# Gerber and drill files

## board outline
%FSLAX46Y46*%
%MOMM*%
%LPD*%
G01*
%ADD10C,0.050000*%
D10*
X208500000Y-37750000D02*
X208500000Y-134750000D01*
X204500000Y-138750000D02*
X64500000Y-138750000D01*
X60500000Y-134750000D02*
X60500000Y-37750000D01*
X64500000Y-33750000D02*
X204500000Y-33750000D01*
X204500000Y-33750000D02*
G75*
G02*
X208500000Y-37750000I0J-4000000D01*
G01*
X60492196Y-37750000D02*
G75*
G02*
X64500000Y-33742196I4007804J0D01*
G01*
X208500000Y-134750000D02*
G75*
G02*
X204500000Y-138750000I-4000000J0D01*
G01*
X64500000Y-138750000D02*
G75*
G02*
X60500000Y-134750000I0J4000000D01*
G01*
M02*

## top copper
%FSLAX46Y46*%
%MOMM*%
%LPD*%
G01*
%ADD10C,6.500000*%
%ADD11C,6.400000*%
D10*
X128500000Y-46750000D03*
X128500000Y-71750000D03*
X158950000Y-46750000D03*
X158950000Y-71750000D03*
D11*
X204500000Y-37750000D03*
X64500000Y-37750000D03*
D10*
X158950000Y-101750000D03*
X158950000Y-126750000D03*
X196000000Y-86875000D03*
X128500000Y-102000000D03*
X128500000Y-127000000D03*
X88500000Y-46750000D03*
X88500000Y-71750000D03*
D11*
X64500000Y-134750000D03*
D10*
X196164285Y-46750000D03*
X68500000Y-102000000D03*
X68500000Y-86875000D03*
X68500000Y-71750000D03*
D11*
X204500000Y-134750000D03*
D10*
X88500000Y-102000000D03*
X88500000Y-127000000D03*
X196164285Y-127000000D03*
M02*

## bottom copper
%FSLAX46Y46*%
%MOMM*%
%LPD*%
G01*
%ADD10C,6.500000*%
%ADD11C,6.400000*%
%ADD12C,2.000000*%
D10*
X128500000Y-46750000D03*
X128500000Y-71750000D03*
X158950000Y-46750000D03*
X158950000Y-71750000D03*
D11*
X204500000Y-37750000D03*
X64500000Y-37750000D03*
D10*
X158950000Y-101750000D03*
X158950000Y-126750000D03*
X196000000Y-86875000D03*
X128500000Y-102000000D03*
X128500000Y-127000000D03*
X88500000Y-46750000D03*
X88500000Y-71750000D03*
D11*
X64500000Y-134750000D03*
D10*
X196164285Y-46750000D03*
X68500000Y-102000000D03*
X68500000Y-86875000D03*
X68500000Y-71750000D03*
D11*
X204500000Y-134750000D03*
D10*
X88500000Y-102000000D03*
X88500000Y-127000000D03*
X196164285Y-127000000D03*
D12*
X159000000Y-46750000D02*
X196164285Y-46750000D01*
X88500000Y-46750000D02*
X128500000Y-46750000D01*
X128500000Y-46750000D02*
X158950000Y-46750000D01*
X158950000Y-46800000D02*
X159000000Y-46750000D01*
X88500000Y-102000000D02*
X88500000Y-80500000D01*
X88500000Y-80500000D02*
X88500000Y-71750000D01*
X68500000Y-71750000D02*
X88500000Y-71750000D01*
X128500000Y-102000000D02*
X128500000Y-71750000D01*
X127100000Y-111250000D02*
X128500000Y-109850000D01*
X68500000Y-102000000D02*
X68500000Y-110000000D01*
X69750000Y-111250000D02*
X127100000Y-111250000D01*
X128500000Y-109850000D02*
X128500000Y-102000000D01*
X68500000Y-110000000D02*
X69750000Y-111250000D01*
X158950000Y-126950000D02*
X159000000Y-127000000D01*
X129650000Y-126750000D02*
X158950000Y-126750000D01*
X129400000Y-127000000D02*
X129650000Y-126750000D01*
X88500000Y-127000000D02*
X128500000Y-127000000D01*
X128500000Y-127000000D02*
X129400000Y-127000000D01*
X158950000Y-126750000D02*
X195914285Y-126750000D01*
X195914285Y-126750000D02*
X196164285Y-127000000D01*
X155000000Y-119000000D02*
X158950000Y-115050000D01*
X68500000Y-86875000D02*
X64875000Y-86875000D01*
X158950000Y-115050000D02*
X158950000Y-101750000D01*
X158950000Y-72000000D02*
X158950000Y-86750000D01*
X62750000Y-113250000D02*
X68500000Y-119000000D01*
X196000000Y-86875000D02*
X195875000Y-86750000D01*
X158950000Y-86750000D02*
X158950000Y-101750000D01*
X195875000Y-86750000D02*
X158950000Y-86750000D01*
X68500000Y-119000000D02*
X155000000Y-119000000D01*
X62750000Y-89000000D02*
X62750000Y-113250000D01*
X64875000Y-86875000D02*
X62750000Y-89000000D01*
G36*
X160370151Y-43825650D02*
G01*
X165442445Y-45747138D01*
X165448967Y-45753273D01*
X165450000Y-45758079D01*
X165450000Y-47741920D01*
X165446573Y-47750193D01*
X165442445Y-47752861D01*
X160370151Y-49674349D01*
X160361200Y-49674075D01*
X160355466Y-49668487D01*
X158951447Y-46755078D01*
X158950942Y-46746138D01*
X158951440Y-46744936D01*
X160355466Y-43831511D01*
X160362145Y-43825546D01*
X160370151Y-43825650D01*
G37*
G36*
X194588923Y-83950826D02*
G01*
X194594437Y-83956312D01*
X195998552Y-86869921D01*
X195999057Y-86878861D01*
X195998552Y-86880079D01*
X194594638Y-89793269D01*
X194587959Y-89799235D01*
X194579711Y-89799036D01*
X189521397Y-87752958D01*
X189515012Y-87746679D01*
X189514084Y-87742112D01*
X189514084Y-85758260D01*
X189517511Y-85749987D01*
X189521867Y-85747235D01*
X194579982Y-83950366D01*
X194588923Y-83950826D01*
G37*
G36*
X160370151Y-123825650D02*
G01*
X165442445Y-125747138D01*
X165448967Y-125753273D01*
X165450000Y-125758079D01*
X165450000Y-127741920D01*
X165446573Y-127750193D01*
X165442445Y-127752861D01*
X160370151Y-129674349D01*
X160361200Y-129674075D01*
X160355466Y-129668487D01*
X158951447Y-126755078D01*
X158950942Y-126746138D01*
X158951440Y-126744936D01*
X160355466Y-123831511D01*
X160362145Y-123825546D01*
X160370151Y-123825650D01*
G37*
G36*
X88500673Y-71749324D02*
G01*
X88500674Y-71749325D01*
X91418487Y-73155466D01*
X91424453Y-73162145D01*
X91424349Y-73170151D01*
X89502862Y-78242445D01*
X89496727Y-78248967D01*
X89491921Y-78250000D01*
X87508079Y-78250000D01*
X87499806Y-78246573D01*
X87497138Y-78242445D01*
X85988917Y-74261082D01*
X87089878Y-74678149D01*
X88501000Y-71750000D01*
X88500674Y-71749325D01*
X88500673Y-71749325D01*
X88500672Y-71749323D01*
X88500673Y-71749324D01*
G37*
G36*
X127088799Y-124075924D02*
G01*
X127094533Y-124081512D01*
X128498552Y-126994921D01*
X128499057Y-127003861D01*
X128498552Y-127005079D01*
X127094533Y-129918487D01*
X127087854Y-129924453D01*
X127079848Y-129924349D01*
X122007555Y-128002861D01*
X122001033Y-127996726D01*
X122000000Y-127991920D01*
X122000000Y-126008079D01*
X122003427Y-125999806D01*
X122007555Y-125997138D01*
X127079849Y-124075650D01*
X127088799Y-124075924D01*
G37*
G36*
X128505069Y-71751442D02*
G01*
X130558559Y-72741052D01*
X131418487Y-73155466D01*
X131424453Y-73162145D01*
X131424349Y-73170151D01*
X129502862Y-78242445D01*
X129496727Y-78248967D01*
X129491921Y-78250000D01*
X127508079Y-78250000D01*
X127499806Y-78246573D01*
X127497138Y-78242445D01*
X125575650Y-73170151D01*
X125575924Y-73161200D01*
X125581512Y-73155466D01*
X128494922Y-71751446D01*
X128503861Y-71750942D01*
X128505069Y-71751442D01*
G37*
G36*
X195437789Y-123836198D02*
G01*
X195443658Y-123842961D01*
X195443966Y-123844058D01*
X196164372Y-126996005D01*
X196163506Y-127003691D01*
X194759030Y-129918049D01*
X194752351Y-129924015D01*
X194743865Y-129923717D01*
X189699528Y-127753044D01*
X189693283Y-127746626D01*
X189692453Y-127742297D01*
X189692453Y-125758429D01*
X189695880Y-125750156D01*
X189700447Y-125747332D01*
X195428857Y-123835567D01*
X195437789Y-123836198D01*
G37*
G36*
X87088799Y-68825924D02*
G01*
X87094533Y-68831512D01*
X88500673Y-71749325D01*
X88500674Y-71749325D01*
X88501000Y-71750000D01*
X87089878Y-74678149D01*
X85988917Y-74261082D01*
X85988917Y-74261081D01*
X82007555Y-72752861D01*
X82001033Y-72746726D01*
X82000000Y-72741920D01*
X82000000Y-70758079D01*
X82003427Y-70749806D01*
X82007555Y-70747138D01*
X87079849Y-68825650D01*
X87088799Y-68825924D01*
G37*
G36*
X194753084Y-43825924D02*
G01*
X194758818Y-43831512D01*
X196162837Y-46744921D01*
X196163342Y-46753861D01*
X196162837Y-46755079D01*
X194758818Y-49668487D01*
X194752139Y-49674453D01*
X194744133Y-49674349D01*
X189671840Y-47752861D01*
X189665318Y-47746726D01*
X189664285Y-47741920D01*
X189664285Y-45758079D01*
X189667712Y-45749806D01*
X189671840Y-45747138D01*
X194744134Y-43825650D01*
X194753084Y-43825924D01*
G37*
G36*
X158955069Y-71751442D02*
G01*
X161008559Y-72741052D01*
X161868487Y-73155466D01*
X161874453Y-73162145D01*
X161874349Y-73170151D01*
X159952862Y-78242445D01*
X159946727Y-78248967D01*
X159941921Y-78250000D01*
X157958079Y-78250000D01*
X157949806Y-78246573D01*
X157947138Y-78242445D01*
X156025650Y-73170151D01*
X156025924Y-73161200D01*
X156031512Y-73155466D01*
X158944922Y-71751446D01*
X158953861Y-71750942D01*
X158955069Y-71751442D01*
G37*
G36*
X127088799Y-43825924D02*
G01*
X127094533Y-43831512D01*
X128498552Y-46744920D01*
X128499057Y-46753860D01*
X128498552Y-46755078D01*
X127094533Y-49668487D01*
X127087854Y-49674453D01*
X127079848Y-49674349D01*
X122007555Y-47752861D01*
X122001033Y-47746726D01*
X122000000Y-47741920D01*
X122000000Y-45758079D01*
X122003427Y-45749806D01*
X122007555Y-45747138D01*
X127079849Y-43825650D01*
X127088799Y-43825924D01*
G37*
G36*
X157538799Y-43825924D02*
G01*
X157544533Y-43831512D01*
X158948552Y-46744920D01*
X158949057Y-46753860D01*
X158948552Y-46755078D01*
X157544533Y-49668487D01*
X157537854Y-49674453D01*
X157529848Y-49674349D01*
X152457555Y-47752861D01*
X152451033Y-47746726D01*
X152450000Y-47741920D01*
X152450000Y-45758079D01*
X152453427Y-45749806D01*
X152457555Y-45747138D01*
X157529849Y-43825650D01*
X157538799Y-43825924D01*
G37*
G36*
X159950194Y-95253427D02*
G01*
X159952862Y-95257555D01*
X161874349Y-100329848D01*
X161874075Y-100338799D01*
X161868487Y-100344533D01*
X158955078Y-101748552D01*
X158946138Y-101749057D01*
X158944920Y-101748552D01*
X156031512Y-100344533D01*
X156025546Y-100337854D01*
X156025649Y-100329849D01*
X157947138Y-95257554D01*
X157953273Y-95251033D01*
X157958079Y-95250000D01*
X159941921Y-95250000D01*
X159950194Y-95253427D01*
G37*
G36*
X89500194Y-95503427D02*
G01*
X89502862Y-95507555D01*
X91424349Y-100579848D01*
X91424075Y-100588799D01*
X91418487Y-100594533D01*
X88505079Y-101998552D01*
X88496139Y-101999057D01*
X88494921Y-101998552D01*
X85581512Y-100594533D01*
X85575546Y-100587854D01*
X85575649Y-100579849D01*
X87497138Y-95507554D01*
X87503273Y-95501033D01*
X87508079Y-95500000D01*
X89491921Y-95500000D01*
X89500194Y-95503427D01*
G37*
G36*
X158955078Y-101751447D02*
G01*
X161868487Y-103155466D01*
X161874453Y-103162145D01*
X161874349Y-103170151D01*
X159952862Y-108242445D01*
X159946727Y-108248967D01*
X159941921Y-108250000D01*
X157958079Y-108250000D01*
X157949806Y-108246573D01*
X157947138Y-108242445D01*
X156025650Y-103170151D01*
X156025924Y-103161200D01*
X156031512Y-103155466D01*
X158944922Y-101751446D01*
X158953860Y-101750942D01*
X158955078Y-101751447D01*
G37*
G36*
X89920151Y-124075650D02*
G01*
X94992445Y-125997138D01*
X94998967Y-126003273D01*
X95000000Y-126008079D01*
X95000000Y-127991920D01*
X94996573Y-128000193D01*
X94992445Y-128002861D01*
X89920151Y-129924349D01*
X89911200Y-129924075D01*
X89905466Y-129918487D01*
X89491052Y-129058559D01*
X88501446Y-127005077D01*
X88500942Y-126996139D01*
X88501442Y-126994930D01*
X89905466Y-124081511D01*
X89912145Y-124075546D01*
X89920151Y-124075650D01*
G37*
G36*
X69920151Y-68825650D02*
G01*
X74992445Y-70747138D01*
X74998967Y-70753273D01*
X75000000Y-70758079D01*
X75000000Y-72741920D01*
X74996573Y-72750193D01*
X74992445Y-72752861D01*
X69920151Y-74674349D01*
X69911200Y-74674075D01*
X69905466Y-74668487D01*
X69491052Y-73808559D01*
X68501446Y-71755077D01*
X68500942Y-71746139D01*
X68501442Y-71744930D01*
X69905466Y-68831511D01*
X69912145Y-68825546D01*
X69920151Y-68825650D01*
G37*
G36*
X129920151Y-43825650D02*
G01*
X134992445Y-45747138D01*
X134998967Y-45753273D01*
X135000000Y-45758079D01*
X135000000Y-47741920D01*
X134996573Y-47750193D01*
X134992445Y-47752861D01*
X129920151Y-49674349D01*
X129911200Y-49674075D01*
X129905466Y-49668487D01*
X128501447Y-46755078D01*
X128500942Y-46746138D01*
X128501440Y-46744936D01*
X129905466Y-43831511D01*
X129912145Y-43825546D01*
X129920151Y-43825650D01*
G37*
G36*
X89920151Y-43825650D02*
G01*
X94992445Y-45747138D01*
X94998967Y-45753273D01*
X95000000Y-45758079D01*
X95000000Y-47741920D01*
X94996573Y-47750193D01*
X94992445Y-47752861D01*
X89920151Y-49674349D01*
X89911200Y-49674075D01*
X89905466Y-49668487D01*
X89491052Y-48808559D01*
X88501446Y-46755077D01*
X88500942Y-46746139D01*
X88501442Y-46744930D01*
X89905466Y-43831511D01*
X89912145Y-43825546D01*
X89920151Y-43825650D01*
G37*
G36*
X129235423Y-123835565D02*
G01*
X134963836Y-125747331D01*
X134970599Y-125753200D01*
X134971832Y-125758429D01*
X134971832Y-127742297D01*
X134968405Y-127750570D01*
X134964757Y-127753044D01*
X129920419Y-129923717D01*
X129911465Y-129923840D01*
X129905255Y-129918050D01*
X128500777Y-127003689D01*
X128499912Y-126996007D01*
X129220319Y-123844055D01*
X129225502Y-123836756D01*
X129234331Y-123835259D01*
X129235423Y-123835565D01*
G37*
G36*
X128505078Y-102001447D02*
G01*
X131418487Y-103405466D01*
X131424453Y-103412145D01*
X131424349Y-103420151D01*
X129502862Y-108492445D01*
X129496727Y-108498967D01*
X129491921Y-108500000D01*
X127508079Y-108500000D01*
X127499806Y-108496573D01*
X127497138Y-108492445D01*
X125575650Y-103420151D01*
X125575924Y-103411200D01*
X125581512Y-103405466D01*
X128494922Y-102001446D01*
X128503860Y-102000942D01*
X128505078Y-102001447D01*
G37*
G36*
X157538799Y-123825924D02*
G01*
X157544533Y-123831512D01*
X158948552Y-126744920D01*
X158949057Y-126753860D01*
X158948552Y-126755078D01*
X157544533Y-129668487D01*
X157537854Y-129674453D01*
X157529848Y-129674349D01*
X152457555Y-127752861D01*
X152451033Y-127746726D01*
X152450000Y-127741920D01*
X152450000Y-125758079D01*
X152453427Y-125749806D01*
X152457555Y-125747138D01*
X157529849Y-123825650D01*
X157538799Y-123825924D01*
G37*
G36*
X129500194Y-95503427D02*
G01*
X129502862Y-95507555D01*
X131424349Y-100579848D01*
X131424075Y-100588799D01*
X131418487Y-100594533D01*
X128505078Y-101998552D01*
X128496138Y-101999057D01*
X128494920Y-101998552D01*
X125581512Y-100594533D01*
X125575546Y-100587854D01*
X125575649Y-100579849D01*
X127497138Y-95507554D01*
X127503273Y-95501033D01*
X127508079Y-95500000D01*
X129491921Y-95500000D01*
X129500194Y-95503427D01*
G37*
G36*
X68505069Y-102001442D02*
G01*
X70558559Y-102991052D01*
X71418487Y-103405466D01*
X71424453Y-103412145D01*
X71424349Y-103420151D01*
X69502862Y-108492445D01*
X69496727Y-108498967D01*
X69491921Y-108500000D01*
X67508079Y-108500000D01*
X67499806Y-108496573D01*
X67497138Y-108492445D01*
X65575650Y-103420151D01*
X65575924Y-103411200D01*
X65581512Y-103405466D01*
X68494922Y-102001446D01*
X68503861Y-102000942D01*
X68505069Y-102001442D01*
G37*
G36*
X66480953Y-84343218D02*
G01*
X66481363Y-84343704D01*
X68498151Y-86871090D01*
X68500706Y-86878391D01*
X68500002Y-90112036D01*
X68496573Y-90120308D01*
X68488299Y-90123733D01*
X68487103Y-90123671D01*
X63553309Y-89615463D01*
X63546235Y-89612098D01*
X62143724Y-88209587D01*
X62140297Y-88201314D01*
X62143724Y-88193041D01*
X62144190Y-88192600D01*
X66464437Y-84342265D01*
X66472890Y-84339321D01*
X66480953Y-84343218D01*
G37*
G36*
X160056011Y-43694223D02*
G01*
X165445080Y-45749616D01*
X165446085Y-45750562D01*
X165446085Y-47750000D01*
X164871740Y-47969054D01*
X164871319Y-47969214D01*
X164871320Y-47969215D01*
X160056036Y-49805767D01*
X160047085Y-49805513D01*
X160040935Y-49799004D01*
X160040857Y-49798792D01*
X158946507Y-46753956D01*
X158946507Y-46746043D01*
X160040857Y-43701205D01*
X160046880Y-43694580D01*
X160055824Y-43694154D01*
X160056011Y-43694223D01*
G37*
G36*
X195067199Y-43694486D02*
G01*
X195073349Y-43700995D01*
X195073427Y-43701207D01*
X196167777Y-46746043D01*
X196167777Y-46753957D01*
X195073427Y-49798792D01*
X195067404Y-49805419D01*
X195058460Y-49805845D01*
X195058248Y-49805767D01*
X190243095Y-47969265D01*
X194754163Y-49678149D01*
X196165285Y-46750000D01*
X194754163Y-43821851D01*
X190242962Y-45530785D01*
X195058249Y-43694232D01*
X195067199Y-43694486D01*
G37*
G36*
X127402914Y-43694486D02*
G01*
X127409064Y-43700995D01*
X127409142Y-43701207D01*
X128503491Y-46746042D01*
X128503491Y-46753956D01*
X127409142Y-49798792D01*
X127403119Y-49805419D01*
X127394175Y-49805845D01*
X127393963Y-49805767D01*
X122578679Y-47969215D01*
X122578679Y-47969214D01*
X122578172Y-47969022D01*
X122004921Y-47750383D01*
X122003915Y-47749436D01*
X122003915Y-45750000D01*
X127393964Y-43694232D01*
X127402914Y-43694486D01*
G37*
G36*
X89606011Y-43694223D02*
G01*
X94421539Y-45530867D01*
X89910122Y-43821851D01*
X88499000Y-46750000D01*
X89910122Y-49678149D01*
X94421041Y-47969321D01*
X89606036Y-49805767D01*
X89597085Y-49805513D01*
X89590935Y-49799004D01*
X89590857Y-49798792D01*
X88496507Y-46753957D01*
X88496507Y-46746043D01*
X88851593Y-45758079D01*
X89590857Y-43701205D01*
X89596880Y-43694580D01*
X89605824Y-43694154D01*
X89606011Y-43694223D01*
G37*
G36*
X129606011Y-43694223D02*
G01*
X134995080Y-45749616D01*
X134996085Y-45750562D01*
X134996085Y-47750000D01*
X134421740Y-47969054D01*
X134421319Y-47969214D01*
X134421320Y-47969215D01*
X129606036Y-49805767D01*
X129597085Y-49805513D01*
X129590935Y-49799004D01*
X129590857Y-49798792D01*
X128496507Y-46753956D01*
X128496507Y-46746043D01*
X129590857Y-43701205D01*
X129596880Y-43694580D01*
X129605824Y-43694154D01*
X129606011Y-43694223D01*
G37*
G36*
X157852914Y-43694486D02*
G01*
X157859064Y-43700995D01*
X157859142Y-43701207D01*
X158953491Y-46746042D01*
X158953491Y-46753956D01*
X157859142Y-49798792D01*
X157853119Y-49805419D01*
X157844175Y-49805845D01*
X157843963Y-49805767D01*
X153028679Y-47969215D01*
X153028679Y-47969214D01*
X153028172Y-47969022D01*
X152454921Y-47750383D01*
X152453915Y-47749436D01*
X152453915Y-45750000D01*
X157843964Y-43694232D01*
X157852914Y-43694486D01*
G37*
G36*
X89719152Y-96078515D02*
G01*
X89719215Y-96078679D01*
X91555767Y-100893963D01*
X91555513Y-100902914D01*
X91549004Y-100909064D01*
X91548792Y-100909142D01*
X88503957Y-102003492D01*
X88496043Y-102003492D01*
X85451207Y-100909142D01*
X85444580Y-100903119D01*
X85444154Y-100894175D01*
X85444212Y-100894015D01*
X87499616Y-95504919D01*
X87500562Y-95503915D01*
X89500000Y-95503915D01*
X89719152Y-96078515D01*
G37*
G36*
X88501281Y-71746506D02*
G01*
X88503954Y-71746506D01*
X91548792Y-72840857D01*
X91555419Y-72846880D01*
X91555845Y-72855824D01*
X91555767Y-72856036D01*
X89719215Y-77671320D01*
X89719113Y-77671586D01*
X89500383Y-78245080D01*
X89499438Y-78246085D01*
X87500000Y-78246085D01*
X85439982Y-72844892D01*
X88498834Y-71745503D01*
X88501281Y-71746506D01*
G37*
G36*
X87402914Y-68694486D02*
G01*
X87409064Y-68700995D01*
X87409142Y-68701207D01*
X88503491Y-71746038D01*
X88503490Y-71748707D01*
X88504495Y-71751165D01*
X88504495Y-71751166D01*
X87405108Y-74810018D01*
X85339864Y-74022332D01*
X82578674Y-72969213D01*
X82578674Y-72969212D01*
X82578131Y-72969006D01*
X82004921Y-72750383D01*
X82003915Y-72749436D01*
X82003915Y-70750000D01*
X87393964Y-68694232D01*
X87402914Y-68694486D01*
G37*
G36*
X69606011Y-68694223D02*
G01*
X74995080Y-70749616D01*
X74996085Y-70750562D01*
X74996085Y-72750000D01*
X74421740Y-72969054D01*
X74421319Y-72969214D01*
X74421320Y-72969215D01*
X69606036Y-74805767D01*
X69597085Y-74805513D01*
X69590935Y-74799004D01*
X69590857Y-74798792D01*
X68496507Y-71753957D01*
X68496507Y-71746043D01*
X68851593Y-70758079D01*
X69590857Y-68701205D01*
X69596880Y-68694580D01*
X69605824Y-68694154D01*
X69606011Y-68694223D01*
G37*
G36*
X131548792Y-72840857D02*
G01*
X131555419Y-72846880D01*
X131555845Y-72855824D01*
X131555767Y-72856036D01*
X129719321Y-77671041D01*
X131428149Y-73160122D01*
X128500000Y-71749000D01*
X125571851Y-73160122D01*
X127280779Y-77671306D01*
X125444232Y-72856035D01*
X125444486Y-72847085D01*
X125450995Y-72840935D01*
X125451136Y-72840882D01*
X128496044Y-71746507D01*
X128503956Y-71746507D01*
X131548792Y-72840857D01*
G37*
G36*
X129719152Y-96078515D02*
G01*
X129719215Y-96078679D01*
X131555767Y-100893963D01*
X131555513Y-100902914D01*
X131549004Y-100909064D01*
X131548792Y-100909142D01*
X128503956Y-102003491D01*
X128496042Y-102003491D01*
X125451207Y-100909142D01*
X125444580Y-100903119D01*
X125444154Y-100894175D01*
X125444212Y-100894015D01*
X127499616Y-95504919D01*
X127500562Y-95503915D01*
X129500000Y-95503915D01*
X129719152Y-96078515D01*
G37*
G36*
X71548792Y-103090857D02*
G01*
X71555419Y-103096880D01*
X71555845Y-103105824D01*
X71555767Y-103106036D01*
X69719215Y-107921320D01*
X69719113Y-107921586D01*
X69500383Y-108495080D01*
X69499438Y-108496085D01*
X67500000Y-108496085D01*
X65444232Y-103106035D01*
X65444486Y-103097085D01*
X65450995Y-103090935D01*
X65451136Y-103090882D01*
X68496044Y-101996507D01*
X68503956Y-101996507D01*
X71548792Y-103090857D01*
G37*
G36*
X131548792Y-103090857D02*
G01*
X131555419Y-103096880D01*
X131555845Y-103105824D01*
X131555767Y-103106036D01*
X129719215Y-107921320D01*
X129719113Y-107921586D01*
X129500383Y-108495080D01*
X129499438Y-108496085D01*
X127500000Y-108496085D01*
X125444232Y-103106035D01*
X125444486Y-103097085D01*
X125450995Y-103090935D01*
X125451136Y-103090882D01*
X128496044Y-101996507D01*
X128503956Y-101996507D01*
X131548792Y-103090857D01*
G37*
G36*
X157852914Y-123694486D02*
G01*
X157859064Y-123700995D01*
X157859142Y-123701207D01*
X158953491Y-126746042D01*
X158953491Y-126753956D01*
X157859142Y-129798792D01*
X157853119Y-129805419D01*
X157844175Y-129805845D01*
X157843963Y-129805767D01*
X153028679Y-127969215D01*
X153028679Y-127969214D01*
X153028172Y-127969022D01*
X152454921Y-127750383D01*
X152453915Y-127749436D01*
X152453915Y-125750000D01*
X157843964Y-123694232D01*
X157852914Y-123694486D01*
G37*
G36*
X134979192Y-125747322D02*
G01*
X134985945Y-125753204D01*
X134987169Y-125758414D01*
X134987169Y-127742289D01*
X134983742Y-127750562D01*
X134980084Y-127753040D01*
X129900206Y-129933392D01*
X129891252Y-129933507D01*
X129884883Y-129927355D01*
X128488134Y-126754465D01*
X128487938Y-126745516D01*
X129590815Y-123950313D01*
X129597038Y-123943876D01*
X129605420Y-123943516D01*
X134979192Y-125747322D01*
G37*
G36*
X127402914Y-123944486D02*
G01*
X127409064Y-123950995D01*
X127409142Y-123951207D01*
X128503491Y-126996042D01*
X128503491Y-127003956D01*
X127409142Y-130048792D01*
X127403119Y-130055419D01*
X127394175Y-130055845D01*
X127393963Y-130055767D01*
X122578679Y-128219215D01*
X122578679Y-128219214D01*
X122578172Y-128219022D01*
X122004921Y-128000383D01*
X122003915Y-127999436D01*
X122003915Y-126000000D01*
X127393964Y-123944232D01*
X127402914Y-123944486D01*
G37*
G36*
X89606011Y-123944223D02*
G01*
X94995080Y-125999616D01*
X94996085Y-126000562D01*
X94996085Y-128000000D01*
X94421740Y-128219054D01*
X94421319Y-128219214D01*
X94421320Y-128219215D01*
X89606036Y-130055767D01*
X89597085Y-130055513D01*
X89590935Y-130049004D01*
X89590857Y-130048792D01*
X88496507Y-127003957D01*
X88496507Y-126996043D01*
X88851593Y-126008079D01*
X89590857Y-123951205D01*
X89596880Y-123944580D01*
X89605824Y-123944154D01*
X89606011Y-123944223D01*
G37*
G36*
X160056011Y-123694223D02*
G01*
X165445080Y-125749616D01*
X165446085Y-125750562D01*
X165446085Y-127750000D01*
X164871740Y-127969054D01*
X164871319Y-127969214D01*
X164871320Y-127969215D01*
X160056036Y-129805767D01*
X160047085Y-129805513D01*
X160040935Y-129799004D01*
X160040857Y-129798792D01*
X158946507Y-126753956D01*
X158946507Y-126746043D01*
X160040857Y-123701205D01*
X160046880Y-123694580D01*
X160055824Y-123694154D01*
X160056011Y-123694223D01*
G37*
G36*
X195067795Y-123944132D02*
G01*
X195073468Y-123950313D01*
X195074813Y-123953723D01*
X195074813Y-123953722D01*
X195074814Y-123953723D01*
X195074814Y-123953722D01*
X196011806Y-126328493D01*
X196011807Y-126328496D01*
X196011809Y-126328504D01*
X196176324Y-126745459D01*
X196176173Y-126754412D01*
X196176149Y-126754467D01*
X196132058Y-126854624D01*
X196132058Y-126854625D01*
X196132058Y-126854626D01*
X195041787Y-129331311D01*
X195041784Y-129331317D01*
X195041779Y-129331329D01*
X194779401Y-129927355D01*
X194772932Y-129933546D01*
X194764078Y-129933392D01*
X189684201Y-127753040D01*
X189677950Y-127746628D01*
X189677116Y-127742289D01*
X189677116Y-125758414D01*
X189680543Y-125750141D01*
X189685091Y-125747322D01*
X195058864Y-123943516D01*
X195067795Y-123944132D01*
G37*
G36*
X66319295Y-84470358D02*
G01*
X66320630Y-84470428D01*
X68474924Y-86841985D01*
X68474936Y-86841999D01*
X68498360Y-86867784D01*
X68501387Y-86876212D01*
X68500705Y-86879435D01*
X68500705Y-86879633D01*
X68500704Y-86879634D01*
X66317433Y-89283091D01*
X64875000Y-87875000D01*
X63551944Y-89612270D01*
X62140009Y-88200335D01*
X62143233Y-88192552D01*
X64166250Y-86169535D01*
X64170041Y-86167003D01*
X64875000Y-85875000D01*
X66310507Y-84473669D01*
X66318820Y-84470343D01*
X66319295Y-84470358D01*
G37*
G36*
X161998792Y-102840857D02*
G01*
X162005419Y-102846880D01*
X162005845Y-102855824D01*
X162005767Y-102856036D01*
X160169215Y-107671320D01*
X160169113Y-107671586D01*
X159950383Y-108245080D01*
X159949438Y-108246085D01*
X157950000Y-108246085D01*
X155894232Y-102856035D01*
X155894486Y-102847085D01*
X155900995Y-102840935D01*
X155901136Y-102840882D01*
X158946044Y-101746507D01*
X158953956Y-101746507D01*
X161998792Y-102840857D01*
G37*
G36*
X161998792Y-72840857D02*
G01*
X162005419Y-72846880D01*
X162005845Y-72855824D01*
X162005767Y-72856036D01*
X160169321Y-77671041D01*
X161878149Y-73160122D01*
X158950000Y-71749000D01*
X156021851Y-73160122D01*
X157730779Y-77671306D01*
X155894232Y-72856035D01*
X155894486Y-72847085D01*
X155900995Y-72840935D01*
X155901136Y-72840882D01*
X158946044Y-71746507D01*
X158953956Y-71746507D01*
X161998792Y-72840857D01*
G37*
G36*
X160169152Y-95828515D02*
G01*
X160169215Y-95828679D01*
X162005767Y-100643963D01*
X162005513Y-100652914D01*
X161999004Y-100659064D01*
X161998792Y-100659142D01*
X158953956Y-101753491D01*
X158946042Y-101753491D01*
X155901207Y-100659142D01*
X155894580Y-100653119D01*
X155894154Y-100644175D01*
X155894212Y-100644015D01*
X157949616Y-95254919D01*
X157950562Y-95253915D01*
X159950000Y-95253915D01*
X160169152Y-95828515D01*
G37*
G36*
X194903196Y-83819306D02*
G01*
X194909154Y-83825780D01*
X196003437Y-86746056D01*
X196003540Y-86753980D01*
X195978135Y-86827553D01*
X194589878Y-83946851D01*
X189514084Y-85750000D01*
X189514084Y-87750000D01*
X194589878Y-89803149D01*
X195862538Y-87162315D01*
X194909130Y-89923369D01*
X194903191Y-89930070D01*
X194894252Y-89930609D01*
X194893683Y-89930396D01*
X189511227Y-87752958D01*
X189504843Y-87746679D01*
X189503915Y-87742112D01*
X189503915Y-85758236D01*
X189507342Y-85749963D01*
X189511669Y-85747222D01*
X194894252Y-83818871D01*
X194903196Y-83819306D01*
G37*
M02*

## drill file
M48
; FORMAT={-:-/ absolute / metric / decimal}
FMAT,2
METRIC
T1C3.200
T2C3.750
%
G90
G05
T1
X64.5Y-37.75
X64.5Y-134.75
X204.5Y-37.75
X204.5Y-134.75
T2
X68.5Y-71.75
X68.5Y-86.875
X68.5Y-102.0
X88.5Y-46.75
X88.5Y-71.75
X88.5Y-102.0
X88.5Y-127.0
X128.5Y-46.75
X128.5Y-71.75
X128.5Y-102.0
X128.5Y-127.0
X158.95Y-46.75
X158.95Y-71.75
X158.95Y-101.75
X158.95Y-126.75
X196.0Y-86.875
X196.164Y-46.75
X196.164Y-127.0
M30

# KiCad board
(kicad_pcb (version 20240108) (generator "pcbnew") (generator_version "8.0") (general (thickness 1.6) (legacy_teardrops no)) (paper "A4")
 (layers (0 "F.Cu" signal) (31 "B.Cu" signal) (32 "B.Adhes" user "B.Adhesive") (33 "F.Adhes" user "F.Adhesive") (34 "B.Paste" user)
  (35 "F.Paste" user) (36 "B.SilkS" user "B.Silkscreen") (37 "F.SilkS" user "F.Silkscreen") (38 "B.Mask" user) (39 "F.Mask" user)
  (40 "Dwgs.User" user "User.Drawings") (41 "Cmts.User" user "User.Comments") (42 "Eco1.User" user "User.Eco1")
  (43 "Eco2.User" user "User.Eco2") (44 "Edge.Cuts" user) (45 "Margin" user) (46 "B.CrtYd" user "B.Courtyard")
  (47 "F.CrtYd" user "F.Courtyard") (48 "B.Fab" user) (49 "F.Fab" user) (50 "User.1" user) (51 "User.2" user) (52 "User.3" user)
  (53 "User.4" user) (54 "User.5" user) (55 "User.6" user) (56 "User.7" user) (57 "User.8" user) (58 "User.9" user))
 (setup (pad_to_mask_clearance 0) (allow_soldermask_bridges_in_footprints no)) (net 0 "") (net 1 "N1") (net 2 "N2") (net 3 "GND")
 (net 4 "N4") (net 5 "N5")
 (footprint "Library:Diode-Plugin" (layer "F.Cu") (at 128.5 59.25)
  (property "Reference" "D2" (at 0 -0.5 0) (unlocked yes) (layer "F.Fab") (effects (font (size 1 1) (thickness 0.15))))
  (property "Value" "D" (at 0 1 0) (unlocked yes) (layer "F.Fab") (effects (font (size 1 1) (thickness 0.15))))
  (pad "1" thru_hole circle (at 0 -12.5) (size 6.5 6.5) (drill 3.75) (layers "*.Cu" "*.Mask") (remove_unused_layers no) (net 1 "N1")
   (teardrops (best_length_ratio 0.5) (max_length 8) (best_width_ratio 1) (max_width 8) (curve_points 0) (filter_ratio 0.9) (enabled yes)
    (allow_two_segments yes) (prefer_zone_connections yes)))
  (pad "2" thru_hole circle (at 0 12.5) (size 6.5 6.5) (drill 3.75) (layers "*.Cu" "*.Mask") (remove_unused_layers no) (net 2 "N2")
   (teardrops (best_length_ratio 0.5) (max_length 8) (best_width_ratio 1) (max_width 8) (curve_points 0) (filter_ratio 0.9) (enabled yes)
    (allow_two_segments yes) (prefer_zone_connections yes))))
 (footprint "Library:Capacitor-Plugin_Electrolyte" (layer "F.Cu") (at 158.95 59.25)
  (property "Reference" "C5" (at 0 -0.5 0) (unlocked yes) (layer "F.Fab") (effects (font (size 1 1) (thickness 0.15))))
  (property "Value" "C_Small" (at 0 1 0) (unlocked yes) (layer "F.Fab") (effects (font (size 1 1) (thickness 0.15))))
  (pad "1" thru_hole circle (at 0 -12.5) (size 6.5 6.5) (drill 3.75) (layers "*.Cu" "*.Mask") (remove_unused_layers no) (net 1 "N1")
   (teardrops (best_length_ratio 0.5) (max_length 8) (best_width_ratio 1) (max_width 8) (curve_points 0) (filter_ratio 0.9) (enabled yes)
    (allow_two_segments yes) (prefer_zone_connections yes)))
  (pad "2" thru_hole circle (at 0 12.5) (size 6.5 6.5) (drill 3.75) (layers "*.Cu" "*.Mask") (remove_unused_layers no) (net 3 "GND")
   (teardrops (best_length_ratio 0.5) (max_length 8) (best_width_ratio 1) (max_width 8) (curve_points 0) (filter_ratio 0.9) (enabled yes)
    (allow_two_segments yes) (prefer_zone_connections yes))))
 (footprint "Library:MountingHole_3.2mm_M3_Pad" (layer "F.Cu") (at 204.5 37.75)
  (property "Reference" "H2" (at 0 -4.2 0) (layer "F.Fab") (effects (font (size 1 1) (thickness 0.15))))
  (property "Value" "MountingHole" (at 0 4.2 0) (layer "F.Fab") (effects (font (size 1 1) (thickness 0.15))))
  (pad "1" thru_hole circle (at 0 0) (size 6.4 6.4) (drill 3.2) (layers "*.Cu" "*.Mask") (remove_unused_layers no)
   (teardrops (best_length_ratio 0.5) (max_length 8) (best_width_ratio 1) (max_width 8) (curve_points 0) (filter_ratio 0.9) (enabled yes)
    (allow_two_segments yes) (prefer_zone_connections yes))))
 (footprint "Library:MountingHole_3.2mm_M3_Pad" (layer "F.Cu") (at 64.5 37.75)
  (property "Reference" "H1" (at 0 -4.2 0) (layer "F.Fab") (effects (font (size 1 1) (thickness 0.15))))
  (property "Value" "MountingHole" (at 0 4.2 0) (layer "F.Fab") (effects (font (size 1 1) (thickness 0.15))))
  (pad "1" thru_hole circle (at 0 0) (size 6.4 6.4) (drill 3.2) (layers "*.Cu" "*.Mask") (remove_unused_layers no)
   (teardrops (best_length_ratio 0.5) (max_length 8) (best_width_ratio 1) (max_width 8) (curve_points 0) (filter_ratio 0.9) (enabled yes)
    (allow_two_segments yes) (prefer_zone_connections yes))))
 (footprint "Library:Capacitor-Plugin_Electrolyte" (layer "F.Cu") (at 158.95 114.25)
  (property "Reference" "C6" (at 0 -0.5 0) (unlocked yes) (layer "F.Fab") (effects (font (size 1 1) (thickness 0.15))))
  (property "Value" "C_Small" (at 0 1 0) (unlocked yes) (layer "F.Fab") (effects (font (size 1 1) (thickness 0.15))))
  (pad "1" thru_hole circle (at 0 -12.5) (size 6.5 6.5) (drill 3.75) (layers "*.Cu" "*.Mask") (remove_unused_layers no) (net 3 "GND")
   (teardrops (best_length_ratio 0.5) (max_length 8) (best_width_ratio 1) (max_width 8) (curve_points 0) (filter_ratio 0.9) (enabled yes)
    (allow_two_segments yes) (prefer_zone_connections yes)))
  (pad "2" thru_hole circle (at 0 12.5) (size 6.5 6.5) (drill 3.75) (layers "*.Cu" "*.Mask") (remove_unused_layers no) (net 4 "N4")
   (teardrops (best_length_ratio 0.5) (max_length 8) (best_width_ratio 1) (max_width 8) (curve_points 0) (filter_ratio 0.9) (enabled yes)
    (allow_two_segments yes) (prefer_zone_connections yes))))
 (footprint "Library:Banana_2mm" (layer "F.Cu") (at 196 86.875)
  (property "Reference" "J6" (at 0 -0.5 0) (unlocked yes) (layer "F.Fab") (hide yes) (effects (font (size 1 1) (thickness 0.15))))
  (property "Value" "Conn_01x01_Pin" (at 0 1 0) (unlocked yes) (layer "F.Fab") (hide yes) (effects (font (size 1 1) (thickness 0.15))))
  (pad "1" thru_hole circle (at 0 0) (size 6.5 6.5) (drill 3.75) (layers "*.Cu" "*.Mask") (remove_unused_layers no) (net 3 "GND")
   (teardrops (best_length_ratio 0.5) (max_length 8) (best_width_ratio 1) (max_width 8) (curve_points 0) (filter_ratio 0.9) (enabled yes)
    (allow_two_segments yes) (prefer_zone_connections yes))))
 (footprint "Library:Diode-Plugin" (layer "F.Cu") (at 128.5 114.5)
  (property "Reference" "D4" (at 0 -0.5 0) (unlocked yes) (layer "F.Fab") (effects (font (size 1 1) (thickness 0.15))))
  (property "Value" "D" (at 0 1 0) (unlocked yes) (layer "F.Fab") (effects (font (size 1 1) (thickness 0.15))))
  (pad "1" thru_hole circle (at 0 -12.5) (size 6.5 6.5) (drill 3.75) (layers "*.Cu" "*.Mask") (remove_unused_layers no) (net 2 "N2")
   (teardrops (best_length_ratio 0.5) (max_length 8) (best_width_ratio 1) (max_width 8) (curve_points 0) (filter_ratio 0.9) (enabled yes)
    (allow_two_segments yes) (prefer_zone_connections yes)))
  (pad "2" thru_hole circle (at 0 12.5) (size 6.5 6.5) (drill 3.75) (layers "*.Cu" "*.Mask") (remove_unused_layers no) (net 4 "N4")
   (teardrops (best_length_ratio 0.5) (max_length 8) (best_width_ratio 1) (max_width 8) (curve_points 0) (filter_ratio 0.9) (enabled yes)
    (allow_two_segments yes) (prefer_zone_connections yes))))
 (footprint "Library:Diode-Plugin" (layer "F.Cu") (at 88.5 59.25)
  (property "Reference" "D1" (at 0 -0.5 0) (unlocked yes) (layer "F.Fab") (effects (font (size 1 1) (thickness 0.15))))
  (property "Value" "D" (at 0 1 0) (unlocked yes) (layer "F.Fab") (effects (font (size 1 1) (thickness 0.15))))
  (pad "1" thru_hole circle (at 0 -12.5) (size 6.5 6.5) (drill 3.75) (layers "*.Cu" "*.Mask") (remove_unused_layers no) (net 1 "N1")
   (teardrops (best_length_ratio 0.5) (max_length 8) (best_width_ratio 1) (max_width 8) (curve_points 0) (filter_ratio 0.9) (enabled yes)
    (allow_two_segments yes) (prefer_zone_connections yes)))
  (pad "2" thru_hole circle (at 0 12.5) (size 6.5 6.5) (drill 3.75) (layers "*.Cu" "*.Mask") (remove_unused_layers no) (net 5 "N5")
   (teardrops (best_length_ratio 0.5) (max_length 8) (best_width_ratio 1) (max_width 8) (curve_points 0) (filter_ratio 0.9) (enabled yes)
    (allow_two_segments yes) (prefer_zone_connections yes))))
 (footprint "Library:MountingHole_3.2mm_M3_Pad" (layer "F.Cu") (at 64.5 134.75)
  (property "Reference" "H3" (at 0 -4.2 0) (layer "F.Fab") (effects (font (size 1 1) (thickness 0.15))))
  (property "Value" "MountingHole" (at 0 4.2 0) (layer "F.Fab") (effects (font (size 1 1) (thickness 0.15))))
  (pad "1" thru_hole circle (at 0 0) (size 6.4 6.4) (drill 3.2) (layers "*.Cu" "*.Mask") (remove_unused_layers no)
   (teardrops (best_length_ratio 0.5) (max_length 8) (best_width_ratio 1) (max_width 8) (curve_points 0) (filter_ratio 0.9) (enabled yes)
    (allow_two_segments yes) (prefer_zone_connections yes))))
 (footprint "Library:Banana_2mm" (layer "F.Cu") (at 196.164285 46.75)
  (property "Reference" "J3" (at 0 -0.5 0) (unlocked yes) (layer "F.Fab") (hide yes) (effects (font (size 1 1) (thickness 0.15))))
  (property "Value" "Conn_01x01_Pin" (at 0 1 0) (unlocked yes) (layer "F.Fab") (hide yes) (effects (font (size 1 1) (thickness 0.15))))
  (pad "1" thru_hole circle (at 0 0) (size 6.5 6.5) (drill 3.75) (layers "*.Cu" "*.Mask") (remove_unused_layers no) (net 1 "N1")
   (teardrops (best_length_ratio 0.5) (max_length 8) (best_width_ratio 1) (max_width 8) (curve_points 0) (filter_ratio 0.9) (enabled yes)
    (allow_two_segments yes) (prefer_zone_connections yes))))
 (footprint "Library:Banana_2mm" (layer "F.Cu") (at 68.5 102)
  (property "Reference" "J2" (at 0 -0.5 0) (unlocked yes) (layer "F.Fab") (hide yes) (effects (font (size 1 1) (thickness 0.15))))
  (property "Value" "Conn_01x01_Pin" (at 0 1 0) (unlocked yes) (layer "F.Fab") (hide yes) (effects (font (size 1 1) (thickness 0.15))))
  (pad "1" thru_hole circle (at 0 0) (size 6.5 6.5) (drill 3.75) (layers "*.Cu" "*.Mask") (remove_unused_layers no) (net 2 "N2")
   (teardrops (best_length_ratio 0.5) (max_length 8) (best_width_ratio 1) (max_width 8) (curve_points 0) (filter_ratio 0.9) (enabled yes)
    (allow_two_segments yes) (prefer_zone_connections yes))))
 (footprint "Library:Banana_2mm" (layer "F.Cu") (at 68.5 86.875)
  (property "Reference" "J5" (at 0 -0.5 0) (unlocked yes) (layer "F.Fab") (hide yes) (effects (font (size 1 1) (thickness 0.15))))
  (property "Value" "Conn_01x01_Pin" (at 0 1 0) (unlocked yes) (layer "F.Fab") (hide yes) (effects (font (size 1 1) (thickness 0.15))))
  (pad "1" thru_hole circle (at 0 0) (size 6.5 6.5) (drill 3.75) (layers "*.Cu" "*.Mask") (remove_unused_layers no) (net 3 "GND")
   (teardrops (best_length_ratio 0.5) (max_length 8) (best_width_ratio 1) (max_width 8) (curve_points 0) (filter_ratio 0.9) (enabled yes)
    (allow_two_segments yes) (prefer_zone_connections yes))))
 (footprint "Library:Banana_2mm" (layer "F.Cu") (at 68.5 71.75)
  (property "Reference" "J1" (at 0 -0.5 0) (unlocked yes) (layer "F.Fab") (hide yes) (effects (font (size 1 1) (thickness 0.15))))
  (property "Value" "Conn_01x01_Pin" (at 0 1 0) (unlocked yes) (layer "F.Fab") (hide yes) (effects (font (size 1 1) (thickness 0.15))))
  (pad "1" thru_hole circle (at 0 0) (size 6.5 6.5) (drill 3.75) (layers "*.Cu" "*.Mask") (remove_unused_layers no) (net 5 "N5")
   (teardrops (best_length_ratio 0.5) (max_length 8) (best_width_ratio 1) (max_width 8) (curve_points 0) (filter_ratio 0.9) (enabled yes)
    (allow_two_segments yes) (prefer_zone_connections yes))))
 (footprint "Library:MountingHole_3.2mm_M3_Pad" (layer "F.Cu") (at 204.5 134.75)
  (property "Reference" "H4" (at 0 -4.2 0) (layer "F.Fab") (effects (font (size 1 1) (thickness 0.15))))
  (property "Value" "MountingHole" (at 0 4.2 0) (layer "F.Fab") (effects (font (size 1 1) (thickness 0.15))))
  (pad "1" thru_hole circle (at 0 0) (size 6.4 6.4) (drill 3.2) (layers "*.Cu" "*.Mask") (remove_unused_layers no)
   (teardrops (best_length_ratio 0.5) (max_length 8) (best_width_ratio 1) (max_width 8) (curve_points 0) (filter_ratio 0.9) (enabled yes)
    (allow_two_segments yes) (prefer_zone_connections yes))))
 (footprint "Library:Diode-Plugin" (layer "F.Cu") (at 88.5 114.5)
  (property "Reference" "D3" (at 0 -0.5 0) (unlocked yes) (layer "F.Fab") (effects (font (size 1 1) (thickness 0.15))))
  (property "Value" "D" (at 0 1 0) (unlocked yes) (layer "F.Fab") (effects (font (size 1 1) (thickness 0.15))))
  (pad "1" thru_hole circle (at 0 -12.5) (size 6.5 6.5) (drill 3.75) (layers "*.Cu" "*.Mask") (remove_unused_layers no) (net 5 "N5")
   (teardrops (best_length_ratio 0.5) (max_length 8) (best_width_ratio 1) (max_width 8) (curve_points 0) (filter_ratio 0.9) (enabled yes)
    (allow_two_segments yes) (prefer_zone_connections yes)))
  (pad "2" thru_hole circle (at 0 12.5) (size 6.5 6.5) (drill 3.75) (layers "*.Cu" "*.Mask") (remove_unused_layers no) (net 4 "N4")
   (teardrops (best_length_ratio 0.5) (max_length 8) (best_width_ratio 1) (max_width 8) (curve_points 0) (filter_ratio 0.9) (enabled yes)
    (allow_two_segments yes) (prefer_zone_connections yes))))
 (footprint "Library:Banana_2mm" (layer "F.Cu") (at 196.164285 127)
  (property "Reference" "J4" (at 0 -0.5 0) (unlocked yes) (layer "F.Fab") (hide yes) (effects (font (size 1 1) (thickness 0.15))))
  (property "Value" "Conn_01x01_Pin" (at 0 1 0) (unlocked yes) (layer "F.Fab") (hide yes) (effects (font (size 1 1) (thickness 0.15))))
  (pad "1" thru_hole circle (at 0 0) (size 6.5 6.5) (drill 3.75) (layers "*.Cu" "*.Mask") (remove_unused_layers no) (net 4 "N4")
   (teardrops (best_length_ratio 0.5) (max_length 8) (best_width_ratio 1) (max_width 8) (curve_points 0) (filter_ratio 0.9) (enabled yes)
    (allow_two_segments yes) (prefer_zone_connections yes))))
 (gr_line (start 208.5 37.75) (end 208.5 134.75) (stroke (width 0.05) (type default)) (layer "Edge.Cuts"))
 (gr_line (start 204.5 138.75) (end 64.5 138.75) (stroke (width 0.05) (type default)) (layer "Edge.Cuts"))
 (gr_line (start 60.5 134.75) (end 60.5 37.75) (stroke (width 0.05) (type default)) (layer "Edge.Cuts"))
 (gr_line (start 64.5 33.75) (end 204.5 33.75) (locked yes) (stroke (width 0.05) (type default)) (layer "Edge.Cuts"))
 (gr_arc (start 204.5 33.75) (mid 207.328427 34.921573) (end 208.5 37.75) (stroke (width 0.05) (type default)) (layer "Edge.Cuts"))
 (gr_arc (start 60.492196 37.75) (mid 61.666055 34.916055) (end 64.5 33.742196) (stroke (width 0.05) (type default)) (layer "Edge.Cuts"))
 (gr_arc (start 208.5 134.75) (mid 207.328427 137.578427) (end 204.5 138.75) (stroke (width 0.05) (type default)) (layer "Edge.Cuts"))
 (gr_arc (start 64.5 138.75) (mid 61.671573 137.578427) (end 60.5 134.75) (stroke (width 0.05) (type default)) (layer "Edge.Cuts"))
 (segment (start 159 46.75) (end 196.164285 46.75) (width 2) (layer "B.Cu") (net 1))
 (segment (start 88.5 46.75) (end 128.5 46.75) (width 2) (layer "B.Cu") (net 1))
 (segment (start 128.5 46.75) (end 158.95 46.75) (width 2) (layer "B.Cu") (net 1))
 (segment (start 158.95 46.8) (end 159 46.75) (width 2) (layer "B.Cu") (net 1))
 (segment (start 88.5 102) (end 88.5 80.5) (width 2) (layer "B.Cu") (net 5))
 (segment (start 88.5 80.5) (end 88.5 71.75) (width 2) (layer "B.Cu") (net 5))
 (segment (start 68.5 71.75) (end 88.5 71.75) (width 2) (layer "B.Cu") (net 5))
 (segment (start 128.5 102) (end 128.5 71.75) (width 2) (layer "B.Cu") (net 2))
 (segment (start 127.1 111.25) (end 128.5 109.85) (width 2) (layer "B.Cu") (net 2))
 (segment (start 68.5 102) (end 68.5 110) (width 2) (layer "B.Cu") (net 2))
 (segment (start 69.75 111.25) (end 127.1 111.25) (width 2) (layer "B.Cu") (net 2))
 (segment (start 128.5 109.85) (end 128.5 102) (width 2) (layer "B.Cu") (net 2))
 (segment (start 68.5 110) (end 69.75 111.25) (width 2) (layer "B.Cu") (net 2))
 (segment (start 158.95 126.95) (end 159 127) (width 2) (layer "B.Cu") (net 4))
 (segment (start 129.65 126.75) (end 158.95 126.75) (width 2) (layer "B.Cu") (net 4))
 (segment (start 129.4 127) (end 129.65 126.75) (width 2) (layer "B.Cu") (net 4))
 (segment (start 88.5 127) (end 128.5 127) (width 2) (layer "B.Cu") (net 4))
 (segment (start 128.5 127) (end 129.4 127) (width 2) (layer "B.Cu") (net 4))
 (segment (start 158.95 126.75) (end 195.914285 126.75) (width 2) (layer "B.Cu") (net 4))
 (segment (start 195.914285 126.75) (end 196.164285 127) (width 2) (layer "B.Cu") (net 4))
 (segment (start 155 119) (end 158.95 115.05) (width 2) (layer "B.Cu") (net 3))
 (segment (start 68.5 86.875) (end 64.875 86.875) (width 2) (layer "B.Cu") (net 3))
 (segment (start 158.95 115.05) (end 158.95 101.75) (width 2) (layer "B.Cu") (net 3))
 (segment (start 158.95 72) (end 158.95 86.75) (width 2) (layer "B.Cu") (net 3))
 (segment (start 62.75 113.25) (end 68.5 119) (width 2) (layer "B.Cu") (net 3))
 (segment (start 196 86.875) (end 195.875 86.75) (width 2) (layer "B.Cu") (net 3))
 (segment (start 158.95 86.75) (end 158.95 101.75) (width 2) (layer "B.Cu") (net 3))
 (segment (start 195.875 86.75) (end 158.95 86.75) (width 2) (layer "B.Cu") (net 3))
 (segment (start 68.5 119) (end 155 119) (width 2) (layer "B.Cu") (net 3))
 (segment (start 62.75 89) (end 62.75 113.25) (width 2) (layer "B.Cu") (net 3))
 (segment (start 64.875 86.875) (end 62.75 89) (width 2) (layer "B.Cu") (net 3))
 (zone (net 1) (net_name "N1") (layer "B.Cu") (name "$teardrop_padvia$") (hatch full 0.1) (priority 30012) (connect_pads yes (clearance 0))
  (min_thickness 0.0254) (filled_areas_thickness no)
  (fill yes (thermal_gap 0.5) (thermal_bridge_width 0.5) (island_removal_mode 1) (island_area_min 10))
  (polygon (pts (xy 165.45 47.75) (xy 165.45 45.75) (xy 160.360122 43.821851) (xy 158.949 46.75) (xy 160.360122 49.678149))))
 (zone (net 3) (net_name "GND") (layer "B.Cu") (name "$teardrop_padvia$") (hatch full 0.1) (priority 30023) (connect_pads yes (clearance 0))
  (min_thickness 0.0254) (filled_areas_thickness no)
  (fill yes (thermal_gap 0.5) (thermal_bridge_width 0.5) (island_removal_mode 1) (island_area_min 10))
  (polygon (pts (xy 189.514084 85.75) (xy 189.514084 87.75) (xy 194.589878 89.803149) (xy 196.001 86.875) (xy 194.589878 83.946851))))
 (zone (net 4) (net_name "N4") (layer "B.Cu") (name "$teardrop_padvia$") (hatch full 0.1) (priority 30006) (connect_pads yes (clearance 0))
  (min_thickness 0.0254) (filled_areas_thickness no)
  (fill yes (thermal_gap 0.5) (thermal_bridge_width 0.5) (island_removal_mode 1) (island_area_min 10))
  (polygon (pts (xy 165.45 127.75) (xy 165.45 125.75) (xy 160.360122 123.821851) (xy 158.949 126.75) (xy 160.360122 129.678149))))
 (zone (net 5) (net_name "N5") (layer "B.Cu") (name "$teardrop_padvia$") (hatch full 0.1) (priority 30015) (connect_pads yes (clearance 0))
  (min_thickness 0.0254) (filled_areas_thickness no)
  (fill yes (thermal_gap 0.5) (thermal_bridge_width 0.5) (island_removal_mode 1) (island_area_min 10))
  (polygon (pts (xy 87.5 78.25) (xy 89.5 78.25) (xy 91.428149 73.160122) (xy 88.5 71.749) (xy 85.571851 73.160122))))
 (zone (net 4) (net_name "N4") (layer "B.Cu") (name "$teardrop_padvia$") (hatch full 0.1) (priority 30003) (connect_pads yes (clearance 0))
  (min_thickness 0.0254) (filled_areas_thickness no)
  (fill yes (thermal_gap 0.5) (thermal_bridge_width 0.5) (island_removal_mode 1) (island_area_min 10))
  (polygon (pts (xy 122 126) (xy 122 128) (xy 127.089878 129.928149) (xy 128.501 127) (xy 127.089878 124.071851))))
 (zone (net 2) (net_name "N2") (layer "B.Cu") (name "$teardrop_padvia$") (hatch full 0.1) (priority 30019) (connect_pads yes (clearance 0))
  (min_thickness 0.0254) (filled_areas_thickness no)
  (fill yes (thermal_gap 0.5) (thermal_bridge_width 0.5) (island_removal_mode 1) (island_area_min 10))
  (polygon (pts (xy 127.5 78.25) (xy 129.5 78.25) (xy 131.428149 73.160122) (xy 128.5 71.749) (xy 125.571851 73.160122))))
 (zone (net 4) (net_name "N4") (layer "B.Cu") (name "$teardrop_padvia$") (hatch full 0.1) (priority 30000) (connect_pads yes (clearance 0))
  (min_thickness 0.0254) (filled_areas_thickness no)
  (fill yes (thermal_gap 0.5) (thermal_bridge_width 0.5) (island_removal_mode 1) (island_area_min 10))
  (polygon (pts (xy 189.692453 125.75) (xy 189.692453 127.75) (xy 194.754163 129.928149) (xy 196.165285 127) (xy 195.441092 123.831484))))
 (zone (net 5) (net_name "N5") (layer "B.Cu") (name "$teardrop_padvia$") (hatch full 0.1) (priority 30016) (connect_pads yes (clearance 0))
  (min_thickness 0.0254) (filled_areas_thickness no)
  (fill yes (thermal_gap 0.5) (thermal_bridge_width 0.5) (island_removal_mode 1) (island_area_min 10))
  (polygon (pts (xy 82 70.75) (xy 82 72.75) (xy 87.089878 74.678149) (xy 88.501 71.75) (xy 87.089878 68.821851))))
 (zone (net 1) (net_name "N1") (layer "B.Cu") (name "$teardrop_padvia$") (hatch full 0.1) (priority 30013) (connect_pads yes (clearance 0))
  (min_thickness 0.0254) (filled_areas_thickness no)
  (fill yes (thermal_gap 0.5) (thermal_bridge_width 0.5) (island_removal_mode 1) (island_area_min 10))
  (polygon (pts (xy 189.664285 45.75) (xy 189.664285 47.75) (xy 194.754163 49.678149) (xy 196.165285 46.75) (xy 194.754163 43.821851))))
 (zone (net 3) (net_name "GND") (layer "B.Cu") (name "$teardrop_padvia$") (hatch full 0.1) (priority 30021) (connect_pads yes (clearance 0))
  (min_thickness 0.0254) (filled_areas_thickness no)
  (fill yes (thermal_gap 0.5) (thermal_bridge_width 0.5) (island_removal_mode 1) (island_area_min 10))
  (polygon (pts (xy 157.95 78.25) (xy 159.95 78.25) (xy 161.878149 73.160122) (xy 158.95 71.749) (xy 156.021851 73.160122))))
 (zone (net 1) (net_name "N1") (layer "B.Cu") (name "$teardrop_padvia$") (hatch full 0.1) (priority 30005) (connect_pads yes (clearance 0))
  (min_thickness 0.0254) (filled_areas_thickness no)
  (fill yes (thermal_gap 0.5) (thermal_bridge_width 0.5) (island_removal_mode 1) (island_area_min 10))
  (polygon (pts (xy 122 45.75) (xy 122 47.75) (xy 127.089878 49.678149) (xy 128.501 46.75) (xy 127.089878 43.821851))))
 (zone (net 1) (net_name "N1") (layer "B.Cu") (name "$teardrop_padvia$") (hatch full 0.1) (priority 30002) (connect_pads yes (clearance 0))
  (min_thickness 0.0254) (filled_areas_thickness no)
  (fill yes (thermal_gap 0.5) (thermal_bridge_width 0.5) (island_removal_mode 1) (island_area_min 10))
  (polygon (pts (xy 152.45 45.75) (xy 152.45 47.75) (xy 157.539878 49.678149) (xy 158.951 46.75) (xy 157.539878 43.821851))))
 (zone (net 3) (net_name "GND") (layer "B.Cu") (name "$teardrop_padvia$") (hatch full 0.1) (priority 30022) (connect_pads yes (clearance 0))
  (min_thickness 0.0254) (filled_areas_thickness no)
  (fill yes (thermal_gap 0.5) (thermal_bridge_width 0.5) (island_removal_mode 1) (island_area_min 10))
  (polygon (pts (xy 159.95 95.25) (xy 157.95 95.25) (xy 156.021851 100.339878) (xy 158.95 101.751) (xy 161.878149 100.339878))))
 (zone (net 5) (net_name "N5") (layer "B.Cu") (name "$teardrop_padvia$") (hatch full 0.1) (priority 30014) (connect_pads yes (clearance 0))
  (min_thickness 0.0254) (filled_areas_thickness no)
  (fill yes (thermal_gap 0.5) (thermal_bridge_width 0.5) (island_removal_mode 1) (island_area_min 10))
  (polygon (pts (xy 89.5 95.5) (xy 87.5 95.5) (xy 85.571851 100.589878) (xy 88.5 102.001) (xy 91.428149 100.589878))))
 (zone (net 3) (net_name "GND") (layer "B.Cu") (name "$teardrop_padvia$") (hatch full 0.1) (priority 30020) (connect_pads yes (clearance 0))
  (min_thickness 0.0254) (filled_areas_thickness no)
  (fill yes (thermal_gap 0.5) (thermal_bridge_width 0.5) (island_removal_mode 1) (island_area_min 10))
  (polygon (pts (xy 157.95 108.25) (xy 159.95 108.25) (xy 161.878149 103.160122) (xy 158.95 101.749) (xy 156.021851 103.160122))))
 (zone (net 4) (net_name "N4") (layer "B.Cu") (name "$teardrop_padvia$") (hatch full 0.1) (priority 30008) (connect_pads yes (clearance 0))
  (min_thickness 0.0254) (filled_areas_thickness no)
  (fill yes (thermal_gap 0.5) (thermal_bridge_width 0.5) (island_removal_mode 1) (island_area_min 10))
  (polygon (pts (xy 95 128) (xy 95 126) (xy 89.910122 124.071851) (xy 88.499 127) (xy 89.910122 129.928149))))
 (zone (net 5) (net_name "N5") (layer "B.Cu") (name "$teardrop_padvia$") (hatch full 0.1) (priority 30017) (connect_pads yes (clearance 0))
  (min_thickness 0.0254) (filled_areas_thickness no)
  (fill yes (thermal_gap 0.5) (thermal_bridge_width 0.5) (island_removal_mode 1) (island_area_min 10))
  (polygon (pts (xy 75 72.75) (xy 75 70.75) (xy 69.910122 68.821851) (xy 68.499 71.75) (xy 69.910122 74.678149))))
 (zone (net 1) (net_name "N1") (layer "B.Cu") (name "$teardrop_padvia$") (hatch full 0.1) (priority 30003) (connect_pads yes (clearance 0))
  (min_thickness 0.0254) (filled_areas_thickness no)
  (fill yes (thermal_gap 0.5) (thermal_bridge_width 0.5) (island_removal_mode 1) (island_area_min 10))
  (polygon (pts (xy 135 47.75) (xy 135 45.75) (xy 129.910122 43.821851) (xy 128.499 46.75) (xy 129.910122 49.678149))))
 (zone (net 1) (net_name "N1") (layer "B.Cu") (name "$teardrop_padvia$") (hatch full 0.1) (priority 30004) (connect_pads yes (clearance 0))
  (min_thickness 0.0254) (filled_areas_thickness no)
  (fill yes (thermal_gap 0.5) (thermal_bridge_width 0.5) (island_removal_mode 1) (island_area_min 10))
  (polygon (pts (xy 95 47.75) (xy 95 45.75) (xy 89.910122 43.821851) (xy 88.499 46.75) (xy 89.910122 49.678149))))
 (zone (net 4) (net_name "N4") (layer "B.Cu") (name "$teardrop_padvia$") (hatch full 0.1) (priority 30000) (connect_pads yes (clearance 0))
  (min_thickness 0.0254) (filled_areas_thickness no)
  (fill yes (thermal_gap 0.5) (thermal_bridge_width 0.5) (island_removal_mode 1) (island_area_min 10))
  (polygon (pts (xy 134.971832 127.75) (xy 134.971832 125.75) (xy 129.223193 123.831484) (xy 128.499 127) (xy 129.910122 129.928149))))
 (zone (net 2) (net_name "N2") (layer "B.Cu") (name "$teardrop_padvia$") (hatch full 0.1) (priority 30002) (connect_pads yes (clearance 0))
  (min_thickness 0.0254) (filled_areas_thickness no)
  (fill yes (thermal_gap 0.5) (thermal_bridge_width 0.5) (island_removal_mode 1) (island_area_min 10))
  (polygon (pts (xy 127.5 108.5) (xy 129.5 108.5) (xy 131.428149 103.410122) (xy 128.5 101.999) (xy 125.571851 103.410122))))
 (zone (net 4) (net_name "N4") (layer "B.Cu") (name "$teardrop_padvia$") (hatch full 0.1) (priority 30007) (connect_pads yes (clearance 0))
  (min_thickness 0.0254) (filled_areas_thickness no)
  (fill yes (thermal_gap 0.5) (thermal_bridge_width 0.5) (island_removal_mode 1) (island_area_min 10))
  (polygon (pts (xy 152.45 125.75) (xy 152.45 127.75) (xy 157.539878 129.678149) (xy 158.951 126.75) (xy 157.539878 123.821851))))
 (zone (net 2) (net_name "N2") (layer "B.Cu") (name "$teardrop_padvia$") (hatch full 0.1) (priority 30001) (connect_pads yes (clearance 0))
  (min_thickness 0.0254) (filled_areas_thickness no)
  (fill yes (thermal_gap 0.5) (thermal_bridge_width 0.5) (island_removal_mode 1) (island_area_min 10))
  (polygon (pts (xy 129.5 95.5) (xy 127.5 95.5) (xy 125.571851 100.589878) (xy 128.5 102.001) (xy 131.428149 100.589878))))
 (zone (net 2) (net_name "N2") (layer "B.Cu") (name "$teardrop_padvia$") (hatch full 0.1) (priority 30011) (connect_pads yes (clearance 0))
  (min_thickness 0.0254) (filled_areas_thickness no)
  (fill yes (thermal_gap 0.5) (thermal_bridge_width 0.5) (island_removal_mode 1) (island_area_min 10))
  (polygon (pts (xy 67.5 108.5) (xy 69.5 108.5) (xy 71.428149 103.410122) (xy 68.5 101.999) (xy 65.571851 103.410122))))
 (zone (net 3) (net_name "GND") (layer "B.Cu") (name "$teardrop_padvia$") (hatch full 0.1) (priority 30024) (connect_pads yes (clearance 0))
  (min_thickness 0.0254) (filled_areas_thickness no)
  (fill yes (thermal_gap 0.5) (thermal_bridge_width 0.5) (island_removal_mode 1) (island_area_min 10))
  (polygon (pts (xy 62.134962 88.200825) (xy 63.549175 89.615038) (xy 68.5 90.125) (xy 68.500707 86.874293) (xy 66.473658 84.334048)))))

